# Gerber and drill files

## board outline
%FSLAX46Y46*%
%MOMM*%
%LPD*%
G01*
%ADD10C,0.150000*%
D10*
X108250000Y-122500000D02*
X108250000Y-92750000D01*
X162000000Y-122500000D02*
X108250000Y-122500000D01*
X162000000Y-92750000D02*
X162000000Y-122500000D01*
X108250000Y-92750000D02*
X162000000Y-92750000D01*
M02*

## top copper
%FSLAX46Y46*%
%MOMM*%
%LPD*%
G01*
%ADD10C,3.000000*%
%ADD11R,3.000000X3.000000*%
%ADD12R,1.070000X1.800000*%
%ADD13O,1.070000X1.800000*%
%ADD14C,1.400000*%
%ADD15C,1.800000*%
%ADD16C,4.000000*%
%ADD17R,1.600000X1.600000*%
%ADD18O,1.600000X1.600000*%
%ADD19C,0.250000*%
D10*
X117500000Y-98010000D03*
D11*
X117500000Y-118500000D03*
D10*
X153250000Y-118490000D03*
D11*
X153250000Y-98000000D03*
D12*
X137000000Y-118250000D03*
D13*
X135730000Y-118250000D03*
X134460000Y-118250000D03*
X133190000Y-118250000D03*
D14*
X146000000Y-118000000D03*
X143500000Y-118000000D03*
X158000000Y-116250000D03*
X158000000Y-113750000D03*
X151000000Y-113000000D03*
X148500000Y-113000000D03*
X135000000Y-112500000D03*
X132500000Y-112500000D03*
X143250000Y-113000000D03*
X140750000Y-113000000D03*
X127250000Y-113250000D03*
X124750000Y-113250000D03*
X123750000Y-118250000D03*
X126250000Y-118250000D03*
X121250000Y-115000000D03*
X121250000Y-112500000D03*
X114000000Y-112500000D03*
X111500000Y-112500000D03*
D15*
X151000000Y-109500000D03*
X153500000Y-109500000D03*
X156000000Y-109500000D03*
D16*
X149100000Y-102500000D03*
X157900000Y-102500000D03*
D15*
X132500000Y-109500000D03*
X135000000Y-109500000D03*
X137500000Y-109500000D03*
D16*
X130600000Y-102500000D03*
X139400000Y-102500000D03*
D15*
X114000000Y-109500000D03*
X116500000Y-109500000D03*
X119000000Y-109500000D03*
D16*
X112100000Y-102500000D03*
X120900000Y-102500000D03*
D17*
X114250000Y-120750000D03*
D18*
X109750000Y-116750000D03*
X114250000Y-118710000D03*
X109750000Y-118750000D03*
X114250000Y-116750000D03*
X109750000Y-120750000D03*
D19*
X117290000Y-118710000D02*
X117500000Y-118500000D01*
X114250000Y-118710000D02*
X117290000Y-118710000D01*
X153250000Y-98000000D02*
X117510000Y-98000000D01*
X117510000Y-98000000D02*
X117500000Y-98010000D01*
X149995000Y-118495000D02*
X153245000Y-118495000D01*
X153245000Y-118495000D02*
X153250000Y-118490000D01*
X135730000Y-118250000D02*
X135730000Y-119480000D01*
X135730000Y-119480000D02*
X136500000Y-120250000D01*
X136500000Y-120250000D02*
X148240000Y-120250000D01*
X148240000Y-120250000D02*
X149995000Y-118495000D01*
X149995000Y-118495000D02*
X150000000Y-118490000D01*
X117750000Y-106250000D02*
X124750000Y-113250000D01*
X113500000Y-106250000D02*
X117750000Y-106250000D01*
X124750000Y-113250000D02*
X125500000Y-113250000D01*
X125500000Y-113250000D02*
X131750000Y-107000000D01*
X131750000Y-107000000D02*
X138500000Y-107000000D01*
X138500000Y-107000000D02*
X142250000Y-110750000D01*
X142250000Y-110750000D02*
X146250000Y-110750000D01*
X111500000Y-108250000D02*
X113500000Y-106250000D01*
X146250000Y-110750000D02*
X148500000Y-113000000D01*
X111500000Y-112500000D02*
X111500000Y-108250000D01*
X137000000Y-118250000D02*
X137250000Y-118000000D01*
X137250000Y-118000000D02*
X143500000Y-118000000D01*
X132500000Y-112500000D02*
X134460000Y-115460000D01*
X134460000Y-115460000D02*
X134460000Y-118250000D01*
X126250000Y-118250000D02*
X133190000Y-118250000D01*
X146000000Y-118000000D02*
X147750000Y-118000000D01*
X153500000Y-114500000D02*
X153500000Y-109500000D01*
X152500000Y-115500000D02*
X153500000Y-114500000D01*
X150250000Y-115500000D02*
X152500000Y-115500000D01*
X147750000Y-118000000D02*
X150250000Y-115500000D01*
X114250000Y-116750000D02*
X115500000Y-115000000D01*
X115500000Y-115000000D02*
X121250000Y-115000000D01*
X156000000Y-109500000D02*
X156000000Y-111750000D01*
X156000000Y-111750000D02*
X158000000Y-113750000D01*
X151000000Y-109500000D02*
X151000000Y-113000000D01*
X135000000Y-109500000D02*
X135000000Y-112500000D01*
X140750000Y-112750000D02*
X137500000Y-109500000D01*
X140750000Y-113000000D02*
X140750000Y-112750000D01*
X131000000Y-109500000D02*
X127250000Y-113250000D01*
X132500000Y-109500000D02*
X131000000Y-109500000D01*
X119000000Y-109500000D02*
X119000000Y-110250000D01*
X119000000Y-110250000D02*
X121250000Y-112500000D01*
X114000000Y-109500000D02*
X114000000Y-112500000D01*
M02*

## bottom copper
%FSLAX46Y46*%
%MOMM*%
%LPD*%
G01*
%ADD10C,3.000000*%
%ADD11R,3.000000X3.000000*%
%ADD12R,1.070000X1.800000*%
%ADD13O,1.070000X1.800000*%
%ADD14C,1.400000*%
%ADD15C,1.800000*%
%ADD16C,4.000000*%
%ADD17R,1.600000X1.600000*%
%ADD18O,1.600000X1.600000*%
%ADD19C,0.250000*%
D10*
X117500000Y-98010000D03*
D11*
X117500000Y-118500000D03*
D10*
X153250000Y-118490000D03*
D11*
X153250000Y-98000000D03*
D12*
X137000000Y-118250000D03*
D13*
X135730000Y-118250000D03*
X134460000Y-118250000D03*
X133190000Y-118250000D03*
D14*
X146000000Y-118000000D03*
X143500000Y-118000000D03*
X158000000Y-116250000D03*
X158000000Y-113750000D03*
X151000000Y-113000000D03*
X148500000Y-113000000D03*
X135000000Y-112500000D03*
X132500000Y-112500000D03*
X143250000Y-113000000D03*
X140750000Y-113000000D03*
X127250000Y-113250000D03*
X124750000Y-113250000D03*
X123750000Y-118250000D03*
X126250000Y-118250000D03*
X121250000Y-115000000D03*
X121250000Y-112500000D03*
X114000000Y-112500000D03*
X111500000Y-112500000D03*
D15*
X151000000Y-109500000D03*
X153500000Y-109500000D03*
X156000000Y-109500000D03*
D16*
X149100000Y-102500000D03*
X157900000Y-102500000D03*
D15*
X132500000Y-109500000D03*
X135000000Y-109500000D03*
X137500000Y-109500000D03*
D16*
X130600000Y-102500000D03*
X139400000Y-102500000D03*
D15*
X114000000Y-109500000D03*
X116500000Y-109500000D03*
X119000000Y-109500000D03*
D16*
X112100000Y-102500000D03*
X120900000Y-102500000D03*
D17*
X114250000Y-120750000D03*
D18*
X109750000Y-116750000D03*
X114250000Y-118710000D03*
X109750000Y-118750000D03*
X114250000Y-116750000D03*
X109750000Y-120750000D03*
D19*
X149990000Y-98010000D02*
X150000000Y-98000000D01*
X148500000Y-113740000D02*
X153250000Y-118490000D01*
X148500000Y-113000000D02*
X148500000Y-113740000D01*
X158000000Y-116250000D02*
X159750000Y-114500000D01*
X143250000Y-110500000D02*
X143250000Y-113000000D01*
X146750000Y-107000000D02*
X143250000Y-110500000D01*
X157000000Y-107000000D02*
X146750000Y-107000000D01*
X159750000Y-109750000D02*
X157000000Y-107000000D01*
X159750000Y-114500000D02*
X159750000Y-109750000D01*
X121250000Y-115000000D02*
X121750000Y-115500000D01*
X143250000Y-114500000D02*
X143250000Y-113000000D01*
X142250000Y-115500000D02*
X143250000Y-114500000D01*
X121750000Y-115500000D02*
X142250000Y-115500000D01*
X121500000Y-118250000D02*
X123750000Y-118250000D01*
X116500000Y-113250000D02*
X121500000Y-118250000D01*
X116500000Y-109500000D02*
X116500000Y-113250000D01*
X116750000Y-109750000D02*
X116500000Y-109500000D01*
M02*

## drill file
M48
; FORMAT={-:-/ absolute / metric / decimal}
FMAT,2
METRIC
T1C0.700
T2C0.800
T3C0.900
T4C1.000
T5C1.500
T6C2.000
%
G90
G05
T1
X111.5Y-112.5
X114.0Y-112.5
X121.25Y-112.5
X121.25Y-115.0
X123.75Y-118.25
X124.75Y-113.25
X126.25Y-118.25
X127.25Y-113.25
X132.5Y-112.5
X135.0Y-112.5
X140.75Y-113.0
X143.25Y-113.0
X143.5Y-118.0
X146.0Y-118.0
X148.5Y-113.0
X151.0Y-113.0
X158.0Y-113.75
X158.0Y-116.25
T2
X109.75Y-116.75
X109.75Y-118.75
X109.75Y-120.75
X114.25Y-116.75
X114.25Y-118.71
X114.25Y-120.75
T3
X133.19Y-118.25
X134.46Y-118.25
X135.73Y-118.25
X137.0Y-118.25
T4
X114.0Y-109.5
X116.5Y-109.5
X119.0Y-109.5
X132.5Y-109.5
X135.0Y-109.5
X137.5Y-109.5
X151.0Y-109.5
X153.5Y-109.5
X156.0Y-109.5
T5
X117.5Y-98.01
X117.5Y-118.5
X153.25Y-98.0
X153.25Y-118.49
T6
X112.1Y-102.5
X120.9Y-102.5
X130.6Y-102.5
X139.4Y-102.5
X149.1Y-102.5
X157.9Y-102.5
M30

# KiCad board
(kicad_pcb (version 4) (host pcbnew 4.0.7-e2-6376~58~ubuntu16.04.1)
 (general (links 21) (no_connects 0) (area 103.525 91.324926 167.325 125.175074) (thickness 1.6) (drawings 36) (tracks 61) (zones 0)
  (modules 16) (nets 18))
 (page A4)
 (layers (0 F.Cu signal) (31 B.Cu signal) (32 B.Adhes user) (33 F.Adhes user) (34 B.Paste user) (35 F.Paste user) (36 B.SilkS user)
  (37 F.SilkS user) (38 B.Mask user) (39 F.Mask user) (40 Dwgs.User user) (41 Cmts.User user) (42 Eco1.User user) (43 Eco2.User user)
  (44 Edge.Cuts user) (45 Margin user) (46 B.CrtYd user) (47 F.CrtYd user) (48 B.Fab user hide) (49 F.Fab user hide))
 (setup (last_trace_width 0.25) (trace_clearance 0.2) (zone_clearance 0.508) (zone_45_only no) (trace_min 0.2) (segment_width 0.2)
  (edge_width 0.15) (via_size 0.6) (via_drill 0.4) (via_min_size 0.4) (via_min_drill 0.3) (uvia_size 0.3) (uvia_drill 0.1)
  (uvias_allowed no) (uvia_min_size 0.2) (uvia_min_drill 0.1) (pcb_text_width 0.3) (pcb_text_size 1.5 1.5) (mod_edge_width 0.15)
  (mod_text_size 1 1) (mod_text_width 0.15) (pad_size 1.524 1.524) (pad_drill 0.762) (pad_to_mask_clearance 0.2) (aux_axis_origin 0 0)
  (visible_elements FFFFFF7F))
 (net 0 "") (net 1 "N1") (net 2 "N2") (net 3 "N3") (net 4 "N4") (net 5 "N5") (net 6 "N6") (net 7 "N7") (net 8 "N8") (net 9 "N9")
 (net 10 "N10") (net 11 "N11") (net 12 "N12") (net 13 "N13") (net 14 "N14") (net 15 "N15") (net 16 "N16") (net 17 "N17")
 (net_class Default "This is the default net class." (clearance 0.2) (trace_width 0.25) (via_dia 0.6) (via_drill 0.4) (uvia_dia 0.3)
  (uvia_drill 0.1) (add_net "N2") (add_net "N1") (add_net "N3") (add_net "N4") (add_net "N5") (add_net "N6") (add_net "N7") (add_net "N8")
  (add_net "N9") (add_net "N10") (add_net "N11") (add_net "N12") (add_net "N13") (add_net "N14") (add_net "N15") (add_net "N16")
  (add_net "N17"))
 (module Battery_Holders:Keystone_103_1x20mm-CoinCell (layer B.Cu) (at 117.5 118.5 90)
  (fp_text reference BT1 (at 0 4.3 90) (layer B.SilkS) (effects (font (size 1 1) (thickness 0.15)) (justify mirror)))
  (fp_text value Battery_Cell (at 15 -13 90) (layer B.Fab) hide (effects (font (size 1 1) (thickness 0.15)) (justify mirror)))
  (pad 2 thru_hole circle (at 20.49 0 90) (size 3 3) (drill 1.5) (layers *.Cu *.Mask) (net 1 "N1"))
  (pad 1 thru_hole rect (at 0 0 90) (size 3 3) (drill 1.5) (layers *.Cu *.Mask) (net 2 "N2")))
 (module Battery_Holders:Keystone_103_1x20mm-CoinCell (layer B.Cu) (at 153.25 98 270)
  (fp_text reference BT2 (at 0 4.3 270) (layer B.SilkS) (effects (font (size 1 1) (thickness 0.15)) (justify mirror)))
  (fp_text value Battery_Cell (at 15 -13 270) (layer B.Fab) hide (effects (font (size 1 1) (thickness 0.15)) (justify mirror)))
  (pad 2 thru_hole circle (at 20.49 0 270) (size 3 3) (drill 1.5) (layers *.Cu *.Mask) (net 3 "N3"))
  (pad 1 thru_hole rect (at 0 0 270) (size 3 3) (drill 1.5) (layers *.Cu *.Mask) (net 1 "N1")))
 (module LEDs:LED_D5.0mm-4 (layer F.Cu) (at 137 118.25 180)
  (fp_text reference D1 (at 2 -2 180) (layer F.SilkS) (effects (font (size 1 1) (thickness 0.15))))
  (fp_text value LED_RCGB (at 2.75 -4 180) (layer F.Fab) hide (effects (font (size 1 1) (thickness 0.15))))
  (pad 1 thru_hole rect (at 0 0 180) (size 1.07 1.8) (drill 0.9) (layers *.Cu *.Mask) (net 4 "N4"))
  (pad 2 thru_hole oval (at 1.27 0 180) (size 1.07 1.8) (drill 0.9) (layers *.Cu *.Mask) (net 3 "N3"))
  (pad 3 thru_hole oval (at 2.54 0 180) (size 1.07 1.8) (drill 0.9) (layers *.Cu *.Mask) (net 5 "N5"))
  (pad 4 thru_hole oval (at 3.81 0 180) (size 1.07 1.8) (drill 0.9) (layers *.Cu *.Mask) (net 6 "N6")))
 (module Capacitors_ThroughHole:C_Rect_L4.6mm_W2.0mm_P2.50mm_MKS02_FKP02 (layer F.Cu) (at 146 118 180)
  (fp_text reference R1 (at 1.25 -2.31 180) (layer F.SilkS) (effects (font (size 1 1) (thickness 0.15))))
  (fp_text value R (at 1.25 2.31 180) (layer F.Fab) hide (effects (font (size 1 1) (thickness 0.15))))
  (pad 1 thru_hole circle (at 0 0 180) (size 1.4 1.4) (drill 0.7) (layers *.Cu *.Mask) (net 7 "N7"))
  (pad 2 thru_hole circle (at 2.5 0 180) (size 1.4 1.4) (drill 0.7) (layers *.Cu *.Mask) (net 4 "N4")))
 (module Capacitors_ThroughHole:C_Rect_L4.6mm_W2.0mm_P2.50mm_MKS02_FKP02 (layer F.Cu) (at 158 116.25 90)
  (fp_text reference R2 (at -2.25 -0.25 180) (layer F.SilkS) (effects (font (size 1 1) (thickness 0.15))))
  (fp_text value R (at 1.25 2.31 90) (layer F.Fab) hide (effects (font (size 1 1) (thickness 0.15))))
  (pad 1 thru_hole circle (at 0 0 90) (size 1.4 1.4) (drill 0.7) (layers *.Cu *.Mask) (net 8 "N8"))
  (pad 2 thru_hole circle (at 2.5 0 90) (size 1.4 1.4) (drill 0.7) (layers *.Cu *.Mask) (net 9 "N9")))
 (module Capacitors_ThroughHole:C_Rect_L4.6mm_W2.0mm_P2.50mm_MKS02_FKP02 (layer F.Cu) (at 151 113 180)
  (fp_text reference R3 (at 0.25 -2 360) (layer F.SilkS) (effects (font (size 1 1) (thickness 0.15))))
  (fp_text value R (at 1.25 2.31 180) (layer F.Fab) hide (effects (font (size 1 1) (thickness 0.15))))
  (pad 1 thru_hole circle (at 0 0 180) (size 1.4 1.4) (drill 0.7) (layers *.Cu *.Mask) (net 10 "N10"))
  (pad 2 thru_hole circle (at 2.5 0 180) (size 1.4 1.4) (drill 0.7) (layers *.Cu *.Mask) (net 3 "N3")))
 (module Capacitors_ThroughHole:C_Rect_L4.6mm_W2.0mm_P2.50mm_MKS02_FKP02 (layer F.Cu) (at 135 112.5 180)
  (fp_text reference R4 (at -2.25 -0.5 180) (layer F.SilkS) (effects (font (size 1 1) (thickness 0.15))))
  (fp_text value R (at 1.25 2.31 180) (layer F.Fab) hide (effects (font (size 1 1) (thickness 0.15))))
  (pad 1 thru_hole circle (at 0 0 180) (size 1.4 1.4) (drill 0.7) (layers *.Cu *.Mask) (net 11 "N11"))
  (pad 2 thru_hole circle (at 2.5 0 180) (size 1.4 1.4) (drill 0.7) (layers *.Cu *.Mask) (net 5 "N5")))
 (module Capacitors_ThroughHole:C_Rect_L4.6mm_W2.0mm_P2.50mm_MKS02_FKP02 (layer F.Cu) (at 143.25 113 180)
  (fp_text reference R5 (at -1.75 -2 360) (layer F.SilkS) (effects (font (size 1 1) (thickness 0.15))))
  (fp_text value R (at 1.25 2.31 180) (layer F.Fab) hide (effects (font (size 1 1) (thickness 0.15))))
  (pad 1 thru_hole circle (at 0 0 180) (size 1.4 1.4) (drill 0.7) (layers *.Cu *.Mask) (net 8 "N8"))
  (pad 2 thru_hole circle (at 2.5 0 180) (size 1.4 1.4) (drill 0.7) (layers *.Cu *.Mask) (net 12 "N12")))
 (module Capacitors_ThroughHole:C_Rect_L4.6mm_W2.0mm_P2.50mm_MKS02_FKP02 (layer F.Cu) (at 127.25 113.25 180)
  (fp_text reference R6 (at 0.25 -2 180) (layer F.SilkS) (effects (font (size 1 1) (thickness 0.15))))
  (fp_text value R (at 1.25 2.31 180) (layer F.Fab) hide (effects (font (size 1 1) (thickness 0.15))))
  (pad 1 thru_hole circle (at 0 0 180) (size 1.4 1.4) (drill 0.7) (layers *.Cu *.Mask) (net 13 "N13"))
  (pad 2 thru_hole circle (at 2.5 0 180) (size 1.4 1.4) (drill 0.7) (layers *.Cu *.Mask) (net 3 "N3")))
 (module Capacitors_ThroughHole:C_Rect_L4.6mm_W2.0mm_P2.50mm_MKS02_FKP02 (layer F.Cu) (at 123.75 118.25)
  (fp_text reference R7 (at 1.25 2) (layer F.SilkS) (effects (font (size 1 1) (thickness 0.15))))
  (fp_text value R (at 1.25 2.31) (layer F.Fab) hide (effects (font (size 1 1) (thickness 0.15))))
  (pad 1 thru_hole circle (at 0 0) (size 1.4 1.4) (drill 0.7) (layers *.Cu *.Mask) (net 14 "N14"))
  (pad 2 thru_hole circle (at 2.5 0) (size 1.4 1.4) (drill 0.7) (layers *.Cu *.Mask) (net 6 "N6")))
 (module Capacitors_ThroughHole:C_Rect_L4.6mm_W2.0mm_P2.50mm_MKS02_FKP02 (layer F.Cu) (at 121.25 115 90)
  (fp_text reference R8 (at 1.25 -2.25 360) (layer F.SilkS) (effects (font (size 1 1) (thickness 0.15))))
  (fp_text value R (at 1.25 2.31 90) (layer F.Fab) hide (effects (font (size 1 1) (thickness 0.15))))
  (pad 1 thru_hole circle (at 0 0 90) (size 1.4 1.4) (drill 0.7) (layers *.Cu *.Mask) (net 8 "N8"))
  (pad 2 thru_hole circle (at 2.5 0 90) (size 1.4 1.4) (drill 0.7) (layers *.Cu *.Mask) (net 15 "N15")))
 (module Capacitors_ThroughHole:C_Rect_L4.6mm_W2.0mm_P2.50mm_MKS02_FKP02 (layer F.Cu) (at 114 112.5 180)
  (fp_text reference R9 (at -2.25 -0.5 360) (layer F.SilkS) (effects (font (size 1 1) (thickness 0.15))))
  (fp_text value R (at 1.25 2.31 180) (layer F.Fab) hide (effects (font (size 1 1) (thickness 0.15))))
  (pad 1 thru_hole circle (at 0 0 180) (size 1.4 1.4) (drill 0.7) (layers *.Cu *.Mask) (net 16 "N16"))
  (pad 2 thru_hole circle (at 2.5 0 180) (size 1.4 1.4) (drill 0.7) (layers *.Cu *.Mask) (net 3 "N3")))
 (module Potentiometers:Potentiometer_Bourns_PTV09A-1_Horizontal (layer F.Cu) (at 156 109.5 90)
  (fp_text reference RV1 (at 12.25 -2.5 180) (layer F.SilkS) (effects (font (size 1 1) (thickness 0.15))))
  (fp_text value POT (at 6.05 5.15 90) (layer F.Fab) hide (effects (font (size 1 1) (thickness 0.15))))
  (pad 3 thru_hole circle (at 0 -5 90) (size 1.8 1.8) (drill 1) (layers *.Cu *.Mask) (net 10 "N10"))
  (pad 2 thru_hole circle (at 0 -2.5 90) (size 1.8 1.8) (drill 1) (layers *.Cu *.Mask) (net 7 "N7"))
  (pad 1 thru_hole circle (at 0 0 90) (size 1.8 1.8) (drill 1) (layers *.Cu *.Mask) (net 9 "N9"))
  (pad 0 np_thru_hole circle (at 7 -6.9 90) (size 4 4) (drill 2) (layers *.Cu *.Mask))
  (pad 0 np_thru_hole circle (at 7 1.9 90) (size 4 4) (drill 2) (layers *.Cu *.Mask)))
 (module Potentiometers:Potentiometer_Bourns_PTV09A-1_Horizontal (layer F.Cu) (at 137.5 109.5 90)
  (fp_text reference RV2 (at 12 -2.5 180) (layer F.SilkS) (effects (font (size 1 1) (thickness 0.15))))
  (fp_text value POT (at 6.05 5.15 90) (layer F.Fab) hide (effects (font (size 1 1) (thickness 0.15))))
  (pad 3 thru_hole circle (at 0 -5 90) (size 1.8 1.8) (drill 1) (layers *.Cu *.Mask) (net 13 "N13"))
  (pad 2 thru_hole circle (at 0 -2.5 90) (size 1.8 1.8) (drill 1) (layers *.Cu *.Mask) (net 11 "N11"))
  (pad 1 thru_hole circle (at 0 0 90) (size 1.8 1.8) (drill 1) (layers *.Cu *.Mask) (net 12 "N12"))
  (pad 0 np_thru_hole circle (at 7 -6.9 90) (size 4 4) (drill 2) (layers *.Cu *.Mask))
  (pad 0 np_thru_hole circle (at 7 1.9 90) (size 4 4) (drill 2) (layers *.Cu *.Mask)))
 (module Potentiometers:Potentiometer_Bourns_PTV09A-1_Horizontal (layer F.Cu) (at 119 109.5 90)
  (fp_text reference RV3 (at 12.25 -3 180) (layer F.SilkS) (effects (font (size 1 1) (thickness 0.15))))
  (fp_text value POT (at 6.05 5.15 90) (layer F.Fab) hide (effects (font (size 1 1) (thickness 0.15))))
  (pad 3 thru_hole circle (at 0 -5 90) (size 1.8 1.8) (drill 1) (layers *.Cu *.Mask) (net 16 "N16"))
  (pad 2 thru_hole circle (at 0 -2.5 90) (size 1.8 1.8) (drill 1) (layers *.Cu *.Mask) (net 14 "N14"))
  (pad 1 thru_hole circle (at 0 0 90) (size 1.8 1.8) (drill 1) (layers *.Cu *.Mask) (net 15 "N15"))
  (pad 0 np_thru_hole circle (at 7 -6.9 90) (size 4 4) (drill 2) (layers *.Cu *.Mask))
  (pad 0 np_thru_hole circle (at 7 1.9 90) (size 4 4) (drill 2) (layers *.Cu *.Mask)))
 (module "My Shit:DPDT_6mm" (layer F.Cu) (at 114.25 120.75 180)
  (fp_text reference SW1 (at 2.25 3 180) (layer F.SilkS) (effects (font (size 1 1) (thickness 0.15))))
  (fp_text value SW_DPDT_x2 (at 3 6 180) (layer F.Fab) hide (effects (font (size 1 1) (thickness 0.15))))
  (pad 1 thru_hole rect (at 0 0 180) (size 1.6 1.6) (drill 0.8) (layers *.Cu *.Mask) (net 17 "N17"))
  (pad 4 thru_hole oval (at 4.5 4 180) (size 1.6 1.6) (drill 0.8) (layers *.Cu *.Mask))
  (pad 2 thru_hole oval (at 0 2.04 180) (size 1.6 1.6) (drill 0.8) (layers *.Cu *.Mask) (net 2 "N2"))
  (pad 5 thru_hole oval (at 4.5 2 180) (size 1.6 1.6) (drill 0.8) (layers *.Cu *.Mask))
  (pad 3 thru_hole oval (at 0 4 180) (size 1.6 1.6) (drill 0.8) (layers *.Cu *.Mask) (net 8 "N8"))
  (pad 6 thru_hole oval (at 4.5 0 180) (size 1.6 1.6) (drill 0.8) (layers *.Cu *.Mask)))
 (gr_line (start 108.25 122.5) (end 108.25 92.75) (angle 90) (layer Edge.Cuts) (width 0.15))
 (gr_line (start 162 122.5) (end 108.25 122.5) (angle 90) (layer Edge.Cuts) (width 0.15))
 (gr_line (start 162 92.75) (end 162 122.5) (angle 90) (layer Edge.Cuts) (width 0.15))
 (gr_line (start 108.25 92.75) (end 162 92.75) (angle 90) (layer Edge.Cuts) (width 0.15))
 (segment (start 149.99 98.01) (end 150 98) (width 0.25) (layer B.Cu) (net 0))
 (segment (start 117.29 118.71) (end 117.5 118.5) (width 0.25) (layer F.Cu) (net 2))
 (segment (start 114.25 118.71) (end 117.29 118.71) (width 0.25) (layer F.Cu) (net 2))
 (segment (start 153.25 98) (end 117.51 98) (width 0.25) (layer F.Cu) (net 1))
 (segment (start 117.51 98) (end 117.5 98.01) (width 0.25) (layer F.Cu) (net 1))
 (segment (start 148.5 113.74) (end 153.25 118.49) (width 0.25) (layer B.Cu) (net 3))
 (segment (start 148.5 113) (end 148.5 113.74) (width 0.25) (layer B.Cu) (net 3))
 (segment (start 149.995 118.495) (end 153.245 118.495) (width 0.25) (layer F.Cu) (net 3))
 (segment (start 153.245 118.495) (end 153.25 118.49) (width 0.25) (layer F.Cu) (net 3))
 (segment (start 135.73 118.25) (end 135.73 119.48) (width 0.25) (layer F.Cu) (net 3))
 (segment (start 135.73 119.48) (end 136.5 120.25) (width 0.25) (layer F.Cu) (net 3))
 (segment (start 136.5 120.25) (end 148.24 120.25) (width 0.25) (layer F.Cu) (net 3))
 (segment (start 148.24 120.25) (end 149.995 118.495) (width 0.25) (layer F.Cu) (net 3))
 (segment (start 149.995 118.495) (end 150 118.49) (width 0.25) (layer F.Cu) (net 3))
 (segment (start 117.75 106.25) (end 124.75 113.25) (width 0.25) (layer F.Cu) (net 3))
 (segment (start 113.5 106.25) (end 117.75 106.25) (width 0.25) (layer F.Cu) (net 3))
 (segment (start 124.75 113.25) (end 125.5 113.25) (width 0.25) (layer F.Cu) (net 3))
 (segment (start 125.5 113.25) (end 131.75 107) (width 0.25) (layer F.Cu) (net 3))
 (segment (start 131.75 107) (end 138.5 107) (width 0.25) (layer F.Cu) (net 3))
 (segment (start 138.5 107) (end 142.25 110.75) (width 0.25) (layer F.Cu) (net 3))
 (segment (start 142.25 110.75) (end 146.25 110.75) (width 0.25) (layer F.Cu) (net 3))
 (segment (start 111.5 108.25) (end 113.5 106.25) (width 0.25) (layer F.Cu) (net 3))
 (segment (start 146.25 110.75) (end 148.5 113) (width 0.25) (layer F.Cu) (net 3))
 (segment (start 111.5 112.5) (end 111.5 108.25) (width 0.25) (layer F.Cu) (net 3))
 (segment (start 137 118.25) (end 137.25 118) (width 0.25) (layer F.Cu) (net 4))
 (segment (start 137.25 118) (end 143.5 118) (width 0.25) (layer F.Cu) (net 4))
 (segment (start 132.5 112.5) (end 134.46 115.46) (width 0.25) (layer F.Cu) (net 5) (status 10))
 (segment (start 134.46 115.46) (end 134.46 118.25) (width 0.25) (layer F.Cu) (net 5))
 (segment (start 126.25 118.25) (end 133.19 118.25) (width 0.25) (layer F.Cu) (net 6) (status 10))
 (segment (start 146 118) (end 147.75 118) (width 0.25) (layer F.Cu) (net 7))
 (segment (start 153.5 114.5) (end 153.5 109.5) (width 0.25) (layer F.Cu) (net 7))
 (segment (start 152.5 115.5) (end 153.5 114.5) (width 0.25) (layer F.Cu) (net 7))
 (segment (start 150.25 115.5) (end 152.5 115.5) (width 0.25) (layer F.Cu) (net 7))
 (segment (start 147.75 118) (end 150.25 115.5) (width 0.25) (layer F.Cu) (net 7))
 (segment (start 114.25 116.75) (end 115.5 115) (width 0.25) (layer F.Cu) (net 8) (status 10))
 (segment (start 115.5 115) (end 121.25 115) (width 0.25) (layer F.Cu) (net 8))
 (segment (start 158 116.25) (end 159.75 114.5) (width 0.25) (layer B.Cu) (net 8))
 (segment (start 143.25 110.5) (end 143.25 113) (width 0.25) (layer B.Cu) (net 8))
 (segment (start 146.75 107) (end 143.25 110.5) (width 0.25) (layer B.Cu) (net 8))
 (segment (start 157 107) (end 146.75 107) (width 0.25) (layer B.Cu) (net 8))
 (segment (start 159.75 109.75) (end 157 107) (width 0.25) (layer B.Cu) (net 8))
 (segment (start 159.75 114.5) (end 159.75 109.75) (width 0.25) (layer B.Cu) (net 8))
 (segment (start 121.25 115) (end 121.75 115.5) (width 0.25) (layer B.Cu) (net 8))
 (segment (start 143.25 114.5) (end 143.25 113) (width 0.25) (layer B.Cu) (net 8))
 (segment (start 142.25 115.5) (end 143.25 114.5) (width 0.25) (layer B.Cu) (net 8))
 (segment (start 121.75 115.5) (end 142.25 115.5) (width 0.25) (layer B.Cu) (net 8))
 (segment (start 156 109.5) (end 156 111.75) (width 0.25) (layer F.Cu) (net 9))
 (segment (start 156 111.75) (end 158 113.75) (width 0.25) (layer F.Cu) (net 9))
 (segment (start 151 109.5) (end 151 113) (width 0.25) (layer F.Cu) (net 10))
 (segment (start 135 109.5) (end 135 112.5) (width 0.25) (layer F.Cu) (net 11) (status 20))
 (segment (start 140.75 112.75) (end 137.5 109.5) (width 0.25) (layer F.Cu) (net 12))
 (segment (start 140.75 113) (end 140.75 112.75) (width 0.25) (layer F.Cu) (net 12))
 (segment (start 131 109.5) (end 127.25 113.25) (width 0.25) (layer F.Cu) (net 13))
 (segment (start 132.5 109.5) (end 131 109.5) (width 0.25) (layer F.Cu) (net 13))
 (segment (start 121.5 118.25) (end 123.75 118.25) (width 0.25) (layer B.Cu) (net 14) (status 20))
 (segment (start 116.5 113.25) (end 121.5 118.25) (width 0.25) (layer B.Cu) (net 14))
 (segment (start 116.5 109.5) (end 116.5 113.25) (width 0.25) (layer B.Cu) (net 14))
 (segment (start 116.75 109.75) (end 116.5 109.5) (width 0.25) (layer B.Cu) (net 14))
 (segment (start 119 109.5) (end 119 110.25) (width 0.25) (layer F.Cu) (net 15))
 (segment (start 119 110.25) (end 121.25 112.5) (width 0.25) (layer F.Cu) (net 15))
 (segment (start 114 109.5) (end 114 112.5) (width 0.25) (layer F.Cu) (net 16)))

